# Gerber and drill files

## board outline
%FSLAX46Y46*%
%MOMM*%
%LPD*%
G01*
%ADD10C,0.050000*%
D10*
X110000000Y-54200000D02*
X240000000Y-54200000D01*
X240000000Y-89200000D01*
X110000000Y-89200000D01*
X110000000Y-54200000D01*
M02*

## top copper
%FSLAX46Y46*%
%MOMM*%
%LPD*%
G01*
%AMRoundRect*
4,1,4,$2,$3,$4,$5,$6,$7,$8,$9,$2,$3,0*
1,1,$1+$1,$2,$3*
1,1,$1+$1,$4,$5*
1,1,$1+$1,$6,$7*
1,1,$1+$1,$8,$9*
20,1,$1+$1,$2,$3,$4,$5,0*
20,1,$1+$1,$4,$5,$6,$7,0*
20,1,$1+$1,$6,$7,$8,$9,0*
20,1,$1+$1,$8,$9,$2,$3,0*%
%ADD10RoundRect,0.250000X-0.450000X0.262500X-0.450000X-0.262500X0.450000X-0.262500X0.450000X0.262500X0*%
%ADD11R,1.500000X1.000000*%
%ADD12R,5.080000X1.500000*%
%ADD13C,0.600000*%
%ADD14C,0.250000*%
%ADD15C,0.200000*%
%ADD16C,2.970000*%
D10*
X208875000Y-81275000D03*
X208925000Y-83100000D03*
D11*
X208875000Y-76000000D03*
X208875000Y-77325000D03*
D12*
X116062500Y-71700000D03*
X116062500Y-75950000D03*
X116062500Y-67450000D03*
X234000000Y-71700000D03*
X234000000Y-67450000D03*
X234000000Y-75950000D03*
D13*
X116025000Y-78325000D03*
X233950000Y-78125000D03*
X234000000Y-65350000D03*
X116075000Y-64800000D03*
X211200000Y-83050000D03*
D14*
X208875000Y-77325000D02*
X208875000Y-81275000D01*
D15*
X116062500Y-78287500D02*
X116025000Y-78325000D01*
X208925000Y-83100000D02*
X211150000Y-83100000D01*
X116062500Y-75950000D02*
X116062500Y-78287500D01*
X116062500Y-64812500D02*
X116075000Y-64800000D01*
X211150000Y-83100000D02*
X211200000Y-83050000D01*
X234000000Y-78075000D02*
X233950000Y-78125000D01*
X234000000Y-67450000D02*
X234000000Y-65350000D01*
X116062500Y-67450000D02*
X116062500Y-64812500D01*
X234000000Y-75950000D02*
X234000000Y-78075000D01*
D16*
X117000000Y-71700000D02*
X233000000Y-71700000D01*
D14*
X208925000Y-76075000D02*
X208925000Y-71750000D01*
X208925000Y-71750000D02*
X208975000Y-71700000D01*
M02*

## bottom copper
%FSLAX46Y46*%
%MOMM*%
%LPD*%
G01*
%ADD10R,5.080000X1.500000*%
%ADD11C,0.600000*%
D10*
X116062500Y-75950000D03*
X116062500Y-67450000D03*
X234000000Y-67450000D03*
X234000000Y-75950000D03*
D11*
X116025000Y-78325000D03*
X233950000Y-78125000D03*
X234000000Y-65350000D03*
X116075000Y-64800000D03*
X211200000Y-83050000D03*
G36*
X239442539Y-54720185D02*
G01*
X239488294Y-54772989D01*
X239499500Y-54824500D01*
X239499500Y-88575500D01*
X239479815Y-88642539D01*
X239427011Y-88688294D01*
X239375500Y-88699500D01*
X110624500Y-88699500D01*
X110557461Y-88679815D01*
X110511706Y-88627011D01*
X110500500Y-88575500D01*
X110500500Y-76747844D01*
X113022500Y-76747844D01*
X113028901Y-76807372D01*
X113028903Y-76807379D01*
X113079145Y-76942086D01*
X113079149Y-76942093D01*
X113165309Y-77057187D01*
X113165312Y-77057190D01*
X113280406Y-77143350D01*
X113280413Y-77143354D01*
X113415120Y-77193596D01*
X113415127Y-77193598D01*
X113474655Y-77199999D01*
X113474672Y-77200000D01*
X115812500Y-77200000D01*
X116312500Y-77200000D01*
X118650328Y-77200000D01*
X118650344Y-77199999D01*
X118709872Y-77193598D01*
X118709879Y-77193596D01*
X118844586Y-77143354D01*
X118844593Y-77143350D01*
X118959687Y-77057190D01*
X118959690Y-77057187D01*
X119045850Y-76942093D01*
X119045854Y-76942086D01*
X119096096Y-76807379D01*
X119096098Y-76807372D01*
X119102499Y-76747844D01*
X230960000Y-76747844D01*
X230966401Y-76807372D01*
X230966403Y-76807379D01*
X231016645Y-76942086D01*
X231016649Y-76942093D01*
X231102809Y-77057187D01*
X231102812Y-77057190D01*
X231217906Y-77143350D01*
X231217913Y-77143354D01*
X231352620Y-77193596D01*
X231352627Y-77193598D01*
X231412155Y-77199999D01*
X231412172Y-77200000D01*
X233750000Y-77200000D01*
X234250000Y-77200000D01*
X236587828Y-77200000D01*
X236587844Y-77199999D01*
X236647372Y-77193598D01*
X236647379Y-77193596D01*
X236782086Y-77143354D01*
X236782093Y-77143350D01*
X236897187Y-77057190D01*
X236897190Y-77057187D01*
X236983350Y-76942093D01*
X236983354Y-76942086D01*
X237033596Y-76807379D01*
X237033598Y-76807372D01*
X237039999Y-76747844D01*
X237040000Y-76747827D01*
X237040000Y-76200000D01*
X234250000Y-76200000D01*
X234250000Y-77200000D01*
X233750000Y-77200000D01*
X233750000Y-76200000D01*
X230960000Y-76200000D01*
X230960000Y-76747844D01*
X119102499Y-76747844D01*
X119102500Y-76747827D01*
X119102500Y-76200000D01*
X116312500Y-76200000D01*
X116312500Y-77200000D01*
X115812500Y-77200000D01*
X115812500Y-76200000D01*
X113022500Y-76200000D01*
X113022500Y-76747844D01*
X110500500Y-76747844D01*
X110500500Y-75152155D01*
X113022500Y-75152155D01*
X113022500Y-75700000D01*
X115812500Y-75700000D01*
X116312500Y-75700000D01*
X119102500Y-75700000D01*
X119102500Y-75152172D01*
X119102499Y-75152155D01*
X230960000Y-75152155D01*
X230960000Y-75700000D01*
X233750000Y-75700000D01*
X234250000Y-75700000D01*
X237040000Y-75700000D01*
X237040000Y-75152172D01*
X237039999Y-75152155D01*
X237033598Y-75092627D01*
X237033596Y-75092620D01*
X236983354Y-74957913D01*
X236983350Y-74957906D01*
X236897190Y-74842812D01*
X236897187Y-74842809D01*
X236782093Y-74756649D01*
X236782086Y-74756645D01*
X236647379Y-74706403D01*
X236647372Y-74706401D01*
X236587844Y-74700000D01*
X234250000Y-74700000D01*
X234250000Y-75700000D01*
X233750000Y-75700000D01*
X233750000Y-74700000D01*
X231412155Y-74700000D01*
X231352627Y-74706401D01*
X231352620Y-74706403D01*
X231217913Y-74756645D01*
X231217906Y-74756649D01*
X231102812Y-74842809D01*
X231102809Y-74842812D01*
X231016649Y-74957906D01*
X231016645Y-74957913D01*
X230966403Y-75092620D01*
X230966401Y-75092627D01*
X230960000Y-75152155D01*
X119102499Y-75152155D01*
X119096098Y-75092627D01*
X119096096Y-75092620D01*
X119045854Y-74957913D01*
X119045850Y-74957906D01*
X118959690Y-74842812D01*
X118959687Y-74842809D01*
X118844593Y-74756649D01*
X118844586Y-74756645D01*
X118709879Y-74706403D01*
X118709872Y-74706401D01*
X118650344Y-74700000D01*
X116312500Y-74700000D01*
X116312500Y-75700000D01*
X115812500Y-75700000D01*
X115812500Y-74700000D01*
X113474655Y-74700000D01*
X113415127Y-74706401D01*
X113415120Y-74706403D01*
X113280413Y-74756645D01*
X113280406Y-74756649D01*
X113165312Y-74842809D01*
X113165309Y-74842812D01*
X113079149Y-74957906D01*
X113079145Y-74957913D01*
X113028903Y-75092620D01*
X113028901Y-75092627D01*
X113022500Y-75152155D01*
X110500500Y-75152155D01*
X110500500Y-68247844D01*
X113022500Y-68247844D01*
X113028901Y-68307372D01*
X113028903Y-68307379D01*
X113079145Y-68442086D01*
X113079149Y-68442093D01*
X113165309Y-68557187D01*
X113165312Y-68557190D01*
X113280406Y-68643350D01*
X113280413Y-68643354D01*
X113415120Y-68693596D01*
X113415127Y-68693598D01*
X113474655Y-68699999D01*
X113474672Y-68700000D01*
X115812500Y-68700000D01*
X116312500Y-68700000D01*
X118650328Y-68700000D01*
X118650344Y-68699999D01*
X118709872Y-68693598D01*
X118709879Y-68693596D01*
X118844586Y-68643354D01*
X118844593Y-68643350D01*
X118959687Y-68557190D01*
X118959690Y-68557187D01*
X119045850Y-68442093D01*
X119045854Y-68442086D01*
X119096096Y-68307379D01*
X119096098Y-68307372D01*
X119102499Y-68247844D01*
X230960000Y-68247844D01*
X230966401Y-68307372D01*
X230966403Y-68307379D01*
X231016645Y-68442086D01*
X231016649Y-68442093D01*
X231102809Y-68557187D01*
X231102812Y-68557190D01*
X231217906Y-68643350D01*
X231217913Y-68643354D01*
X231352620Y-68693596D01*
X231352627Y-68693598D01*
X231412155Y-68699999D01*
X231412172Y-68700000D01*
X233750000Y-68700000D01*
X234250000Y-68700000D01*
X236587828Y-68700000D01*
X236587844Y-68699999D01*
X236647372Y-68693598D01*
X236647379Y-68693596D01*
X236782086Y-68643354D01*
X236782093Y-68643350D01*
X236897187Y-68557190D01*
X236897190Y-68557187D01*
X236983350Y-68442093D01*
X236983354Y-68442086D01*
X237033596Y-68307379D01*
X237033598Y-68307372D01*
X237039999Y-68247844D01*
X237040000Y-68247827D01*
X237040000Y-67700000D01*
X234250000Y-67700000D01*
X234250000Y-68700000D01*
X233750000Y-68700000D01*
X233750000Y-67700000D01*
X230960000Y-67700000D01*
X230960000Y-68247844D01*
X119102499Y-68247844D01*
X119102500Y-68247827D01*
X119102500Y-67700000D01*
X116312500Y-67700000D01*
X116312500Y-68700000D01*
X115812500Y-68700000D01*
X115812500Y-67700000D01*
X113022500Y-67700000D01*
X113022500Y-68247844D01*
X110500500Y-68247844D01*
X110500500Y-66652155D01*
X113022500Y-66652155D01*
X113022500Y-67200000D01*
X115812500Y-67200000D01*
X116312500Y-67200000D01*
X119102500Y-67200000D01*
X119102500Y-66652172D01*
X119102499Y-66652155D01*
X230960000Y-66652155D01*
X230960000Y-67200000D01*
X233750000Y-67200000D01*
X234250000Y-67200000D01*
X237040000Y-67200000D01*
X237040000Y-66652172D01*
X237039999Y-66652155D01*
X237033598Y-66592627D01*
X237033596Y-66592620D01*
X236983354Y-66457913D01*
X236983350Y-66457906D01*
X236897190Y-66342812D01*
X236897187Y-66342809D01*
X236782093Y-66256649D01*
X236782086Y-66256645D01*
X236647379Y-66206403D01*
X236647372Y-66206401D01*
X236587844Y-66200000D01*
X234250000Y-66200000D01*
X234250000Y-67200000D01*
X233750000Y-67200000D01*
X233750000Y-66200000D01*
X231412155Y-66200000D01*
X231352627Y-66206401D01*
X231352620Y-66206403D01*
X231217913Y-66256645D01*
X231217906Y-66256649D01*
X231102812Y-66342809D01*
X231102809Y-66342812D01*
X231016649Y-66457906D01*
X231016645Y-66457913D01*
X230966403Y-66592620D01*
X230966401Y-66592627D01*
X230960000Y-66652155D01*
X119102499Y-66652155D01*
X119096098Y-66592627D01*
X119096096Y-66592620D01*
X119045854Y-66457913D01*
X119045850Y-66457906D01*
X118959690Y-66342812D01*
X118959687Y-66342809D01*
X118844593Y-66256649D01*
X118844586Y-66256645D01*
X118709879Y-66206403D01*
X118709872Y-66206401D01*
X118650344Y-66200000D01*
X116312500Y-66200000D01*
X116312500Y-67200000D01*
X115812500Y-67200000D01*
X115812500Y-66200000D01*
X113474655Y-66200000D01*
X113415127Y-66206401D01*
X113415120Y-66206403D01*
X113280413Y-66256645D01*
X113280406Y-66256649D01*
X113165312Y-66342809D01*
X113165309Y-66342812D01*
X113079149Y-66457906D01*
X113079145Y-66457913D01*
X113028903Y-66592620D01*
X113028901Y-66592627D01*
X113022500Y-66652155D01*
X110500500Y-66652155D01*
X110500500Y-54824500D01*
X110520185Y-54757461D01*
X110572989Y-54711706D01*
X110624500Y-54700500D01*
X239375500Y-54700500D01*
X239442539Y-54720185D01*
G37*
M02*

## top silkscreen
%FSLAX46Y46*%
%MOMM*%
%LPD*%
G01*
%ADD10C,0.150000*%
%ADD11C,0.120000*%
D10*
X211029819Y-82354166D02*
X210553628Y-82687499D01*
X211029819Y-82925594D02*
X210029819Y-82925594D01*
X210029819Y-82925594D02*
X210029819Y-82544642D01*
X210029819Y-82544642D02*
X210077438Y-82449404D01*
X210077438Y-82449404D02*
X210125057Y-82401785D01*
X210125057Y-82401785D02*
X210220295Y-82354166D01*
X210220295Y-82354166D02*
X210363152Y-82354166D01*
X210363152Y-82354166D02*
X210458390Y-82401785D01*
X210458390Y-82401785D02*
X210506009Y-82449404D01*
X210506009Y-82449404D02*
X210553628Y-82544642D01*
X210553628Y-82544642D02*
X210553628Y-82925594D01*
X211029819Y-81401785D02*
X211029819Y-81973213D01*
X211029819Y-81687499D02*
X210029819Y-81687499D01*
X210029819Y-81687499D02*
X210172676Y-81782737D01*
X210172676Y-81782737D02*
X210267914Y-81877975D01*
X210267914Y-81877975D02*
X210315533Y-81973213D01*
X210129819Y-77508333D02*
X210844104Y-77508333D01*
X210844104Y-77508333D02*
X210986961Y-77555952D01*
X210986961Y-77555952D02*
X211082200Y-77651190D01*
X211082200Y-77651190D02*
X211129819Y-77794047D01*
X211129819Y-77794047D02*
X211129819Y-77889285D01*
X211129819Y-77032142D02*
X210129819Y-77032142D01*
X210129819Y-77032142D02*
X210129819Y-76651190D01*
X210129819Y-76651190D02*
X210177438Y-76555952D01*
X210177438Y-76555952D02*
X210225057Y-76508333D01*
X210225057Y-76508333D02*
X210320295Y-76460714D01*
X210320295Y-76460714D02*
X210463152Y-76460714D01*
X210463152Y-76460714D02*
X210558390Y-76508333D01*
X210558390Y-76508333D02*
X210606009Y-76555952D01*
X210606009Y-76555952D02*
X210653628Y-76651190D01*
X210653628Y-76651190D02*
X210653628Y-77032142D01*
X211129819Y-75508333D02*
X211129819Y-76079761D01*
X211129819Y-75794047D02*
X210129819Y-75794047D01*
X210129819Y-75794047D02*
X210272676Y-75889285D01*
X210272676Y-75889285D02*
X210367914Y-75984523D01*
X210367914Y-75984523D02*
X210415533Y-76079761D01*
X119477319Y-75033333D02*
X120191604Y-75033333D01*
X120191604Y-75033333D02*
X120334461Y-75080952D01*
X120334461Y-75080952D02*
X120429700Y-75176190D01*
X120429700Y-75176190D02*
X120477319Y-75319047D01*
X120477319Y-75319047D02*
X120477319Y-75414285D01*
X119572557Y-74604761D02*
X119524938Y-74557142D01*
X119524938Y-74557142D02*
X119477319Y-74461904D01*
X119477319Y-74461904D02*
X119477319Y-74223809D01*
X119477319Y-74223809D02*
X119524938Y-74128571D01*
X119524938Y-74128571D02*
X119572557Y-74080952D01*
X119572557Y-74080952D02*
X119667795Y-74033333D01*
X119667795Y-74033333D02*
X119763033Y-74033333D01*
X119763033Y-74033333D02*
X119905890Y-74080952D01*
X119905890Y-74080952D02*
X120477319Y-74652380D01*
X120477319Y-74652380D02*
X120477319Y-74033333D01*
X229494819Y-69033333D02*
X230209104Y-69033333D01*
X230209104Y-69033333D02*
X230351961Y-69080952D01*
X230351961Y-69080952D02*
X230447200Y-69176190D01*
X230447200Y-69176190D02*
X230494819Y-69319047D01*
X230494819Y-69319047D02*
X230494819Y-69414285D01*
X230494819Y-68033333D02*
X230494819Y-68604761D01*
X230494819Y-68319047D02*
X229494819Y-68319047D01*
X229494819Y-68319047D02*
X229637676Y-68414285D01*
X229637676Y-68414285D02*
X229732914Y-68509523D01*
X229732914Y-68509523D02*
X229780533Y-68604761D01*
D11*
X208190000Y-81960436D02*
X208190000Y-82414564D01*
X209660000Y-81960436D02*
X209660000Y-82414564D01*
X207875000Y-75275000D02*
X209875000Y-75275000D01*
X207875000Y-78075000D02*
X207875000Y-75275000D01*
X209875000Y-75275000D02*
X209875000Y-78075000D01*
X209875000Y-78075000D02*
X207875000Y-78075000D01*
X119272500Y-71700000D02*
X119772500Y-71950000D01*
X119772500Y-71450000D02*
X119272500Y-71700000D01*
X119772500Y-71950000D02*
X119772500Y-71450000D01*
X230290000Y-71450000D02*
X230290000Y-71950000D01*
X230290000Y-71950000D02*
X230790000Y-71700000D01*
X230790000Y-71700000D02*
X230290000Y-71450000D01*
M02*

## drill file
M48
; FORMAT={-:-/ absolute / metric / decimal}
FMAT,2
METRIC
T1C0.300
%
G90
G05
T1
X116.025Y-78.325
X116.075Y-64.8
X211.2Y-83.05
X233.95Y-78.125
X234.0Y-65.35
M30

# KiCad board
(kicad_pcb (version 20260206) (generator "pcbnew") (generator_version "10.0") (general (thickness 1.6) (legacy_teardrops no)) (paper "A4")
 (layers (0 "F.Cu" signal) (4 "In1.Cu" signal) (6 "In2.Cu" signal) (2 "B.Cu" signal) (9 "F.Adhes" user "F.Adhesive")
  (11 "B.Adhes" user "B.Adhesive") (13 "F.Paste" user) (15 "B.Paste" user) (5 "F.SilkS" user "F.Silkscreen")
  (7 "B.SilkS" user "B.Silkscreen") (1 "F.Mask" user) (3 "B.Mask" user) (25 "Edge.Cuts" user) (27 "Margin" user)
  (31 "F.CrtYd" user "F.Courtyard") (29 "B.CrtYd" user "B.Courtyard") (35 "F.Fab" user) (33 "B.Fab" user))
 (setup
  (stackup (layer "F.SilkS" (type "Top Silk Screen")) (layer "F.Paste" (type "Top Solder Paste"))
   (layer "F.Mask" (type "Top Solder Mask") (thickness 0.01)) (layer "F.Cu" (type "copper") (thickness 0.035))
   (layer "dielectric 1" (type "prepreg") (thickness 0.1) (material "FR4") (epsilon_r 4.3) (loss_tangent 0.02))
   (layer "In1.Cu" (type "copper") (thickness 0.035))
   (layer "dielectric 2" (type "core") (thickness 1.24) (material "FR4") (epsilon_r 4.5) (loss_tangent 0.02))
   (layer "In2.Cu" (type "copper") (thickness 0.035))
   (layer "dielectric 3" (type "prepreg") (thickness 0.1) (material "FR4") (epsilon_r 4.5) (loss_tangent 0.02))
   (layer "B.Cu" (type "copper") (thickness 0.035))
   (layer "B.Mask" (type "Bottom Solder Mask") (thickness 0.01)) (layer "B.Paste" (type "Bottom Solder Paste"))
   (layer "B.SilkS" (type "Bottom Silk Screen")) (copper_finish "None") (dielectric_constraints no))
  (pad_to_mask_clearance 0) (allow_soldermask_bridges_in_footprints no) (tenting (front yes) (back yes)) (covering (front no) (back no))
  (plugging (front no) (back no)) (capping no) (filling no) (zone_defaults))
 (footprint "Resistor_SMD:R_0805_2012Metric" (layer "F.Cu") (at 208.925 82.1875 -90)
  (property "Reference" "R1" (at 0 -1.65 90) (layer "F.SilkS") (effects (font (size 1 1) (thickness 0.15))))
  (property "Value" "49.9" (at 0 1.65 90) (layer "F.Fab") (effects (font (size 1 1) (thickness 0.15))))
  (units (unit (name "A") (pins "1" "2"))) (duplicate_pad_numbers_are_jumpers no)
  (fp_line (start -0.227064 0.735) (end 0.227064 0.735) (stroke (width 0.12) (type solid)) (layer "F.SilkS"))
  (fp_line (start -0.227064 -0.735) (end 0.227064 -0.735) (stroke (width 0.12) (type solid)) (layer "F.SilkS"))
  (pad "1" smd roundrect (at -0.9125 0.05 270) (size 1.025 1.4) (layers "F.Cu" "F.Mask" "F.Paste") (roundrect_rratio 0.243902)
   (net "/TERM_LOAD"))
  (pad "2" smd roundrect (at 0.9125 0 270) (size 1.025 1.4) (layers "F.Cu" "F.Mask" "F.Paste") (roundrect_rratio 0.243902) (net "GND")))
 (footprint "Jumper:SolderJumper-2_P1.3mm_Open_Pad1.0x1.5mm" (layer "F.Cu") (at 208.875 76.675 -90)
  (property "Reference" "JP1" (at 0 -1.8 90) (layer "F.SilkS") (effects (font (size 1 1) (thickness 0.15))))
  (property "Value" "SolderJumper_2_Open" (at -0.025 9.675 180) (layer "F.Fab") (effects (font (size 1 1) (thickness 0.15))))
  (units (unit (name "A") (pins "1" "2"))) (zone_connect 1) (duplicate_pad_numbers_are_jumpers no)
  (fp_line (start -1.4 1) (end -1.4 -1) (stroke (width 0.12) (type solid)) (layer "F.SilkS"))
  (fp_line (start 1.4 1) (end -1.4 1) (stroke (width 0.12) (type solid)) (layer "F.SilkS"))
  (fp_line (start -1.4 -1) (end 1.4 -1) (stroke (width 0.12) (type solid)) (layer "F.SilkS"))
  (fp_line (start 1.4 -1) (end 1.4 1) (stroke (width 0.12) (type solid)) (layer "F.SilkS"))
  (pad "1" smd rect (at -0.675 0 270) (size 1 1.5) (layers "F.Cu" "F.Mask") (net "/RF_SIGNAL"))
  (pad "2" smd rect (at 0.65 0 270) (size 1 1.5) (layers "F.Cu" "F.Mask") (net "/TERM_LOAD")))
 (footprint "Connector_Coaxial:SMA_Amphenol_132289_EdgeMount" (layer "F.Cu") (at 116.0625 71.7 180)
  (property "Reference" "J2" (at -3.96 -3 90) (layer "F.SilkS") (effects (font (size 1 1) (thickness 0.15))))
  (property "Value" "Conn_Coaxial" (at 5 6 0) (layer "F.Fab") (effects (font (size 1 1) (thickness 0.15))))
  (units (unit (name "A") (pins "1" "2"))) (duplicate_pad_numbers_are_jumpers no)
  (fp_line (start -3.21 0) (end -3.71 -0.25) (stroke (width 0.12) (type solid)) (layer "F.SilkS"))
  (fp_line (start -3.71 0.25) (end -3.21 0) (stroke (width 0.12) (type solid)) (layer "F.SilkS"))
  (fp_line (start -3.71 -0.25) (end -3.71 0.25) (stroke (width 0.12) (type solid)) (layer "F.SilkS"))
  (pad "1" smd rect (at 0 0 270) (size 1.5 5.08) (layers "F.Cu" "F.Mask" "F.Paste") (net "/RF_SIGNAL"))
  (pad "2" smd rect (at 0 -4.25 270) (size 1.5 5.08) (layers "F.Cu" "F.Mask" "F.Paste") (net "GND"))
  (pad "2" smd rect (at 0 -4.25 270) (size 1.5 5.08) (layers "B.Cu" "B.Mask" "B.Paste") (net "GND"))
  (pad "2" smd rect (at 0 4.25 270) (size 1.5 5.08) (layers "F.Cu" "F.Mask" "F.Paste") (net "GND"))
  (pad "2" smd rect (at 0 4.25 270) (size 1.5 5.08) (layers "B.Cu" "B.Mask" "B.Paste") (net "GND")))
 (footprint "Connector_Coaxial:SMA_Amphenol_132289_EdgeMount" (layer "F.Cu") (at 234 71.7)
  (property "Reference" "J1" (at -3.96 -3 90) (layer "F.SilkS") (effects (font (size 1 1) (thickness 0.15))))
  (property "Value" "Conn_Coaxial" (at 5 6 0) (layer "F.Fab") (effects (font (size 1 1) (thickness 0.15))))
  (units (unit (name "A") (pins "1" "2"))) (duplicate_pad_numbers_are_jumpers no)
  (fp_line (start -3.71 -0.25) (end -3.71 0.25) (stroke (width 0.12) (type solid)) (layer "F.SilkS"))
  (fp_line (start -3.71 0.25) (end -3.21 0) (stroke (width 0.12) (type solid)) (layer "F.SilkS"))
  (fp_line (start -3.21 0) (end -3.71 -0.25) (stroke (width 0.12) (type solid)) (layer "F.SilkS"))
  (pad "1" smd rect (at 0 0 90) (size 1.5 5.08) (layers "F.Cu" "F.Mask" "F.Paste") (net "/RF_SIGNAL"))
  (pad "2" smd rect (at 0 -4.25 90) (size 1.5 5.08) (layers "F.Cu" "F.Mask" "F.Paste") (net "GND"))
  (pad "2" smd rect (at 0 -4.25 90) (size 1.5 5.08) (layers "B.Cu" "B.Mask" "B.Paste") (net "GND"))
  (pad "2" smd rect (at 0 4.25 90) (size 1.5 5.08) (layers "F.Cu" "F.Mask" "F.Paste") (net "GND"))
  (pad "2" smd rect (at 0 4.25 90) (size 1.5 5.08) (layers "B.Cu" "B.Mask" "B.Paste") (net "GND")))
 (gr_rect (start 110 54.2) (end 240 89.2) (stroke (width 0.05) (type solid)) (fill no) (layer "Edge.Cuts"))
 (segment (start 208.875 77.325) (end 208.875 81.275) (width 0.25) (layer "F.Cu") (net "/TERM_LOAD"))
 (segment (start 116.0625 78.2875) (end 116.025 78.325) (width 0.2) (layer "F.Cu") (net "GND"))
 (segment (start 208.925 83.1) (end 211.15 83.1) (width 0.2) (layer "F.Cu") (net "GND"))
 (segment (start 116.0625 75.95) (end 116.0625 78.2875) (width 0.2) (layer "F.Cu") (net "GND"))
 (segment (start 116.0625 64.8125) (end 116.075 64.8) (width 0.2) (layer "F.Cu") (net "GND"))
 (segment (start 211.15 83.1) (end 211.2 83.05) (width 0.2) (layer "F.Cu") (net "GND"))
 (segment (start 234 78.075) (end 233.95 78.125) (width 0.2) (layer "F.Cu") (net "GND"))
 (segment (start 234 67.45) (end 234 65.35) (width 0.2) (layer "F.Cu") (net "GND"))
 (segment (start 116.0625 67.45) (end 116.0625 64.8125) (width 0.2) (layer "F.Cu") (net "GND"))
 (segment (start 234 75.95) (end 234 78.075) (width 0.2) (layer "F.Cu") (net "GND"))
 (via (at 116.025 78.325) (size 0.6) (drill 0.3) (layers "F.Cu" "B.Cu") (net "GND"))
 (via (at 233.95 78.125) (size 0.6) (drill 0.3) (layers "F.Cu" "B.Cu") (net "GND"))
 (via (at 234 65.35) (size 0.6) (drill 0.3) (layers "F.Cu" "B.Cu") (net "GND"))
 (via (at 116.075 64.8) (size 0.6) (drill 0.3) (layers "F.Cu" "B.Cu") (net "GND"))
 (via (at 211.2 83.05) (size 0.6) (drill 0.3) (layers "F.Cu" "B.Cu") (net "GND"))
 (segment (start 117 71.7) (end 233 71.7) (width 2.97) (layer "F.Cu") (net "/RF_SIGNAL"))
 (segment (start 208.925 76.075) (end 208.925 71.75) (width 0.25) (layer "F.Cu") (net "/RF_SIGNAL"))
 (segment (start 208.925 71.75) (end 208.975 71.7) (width 0.25) (layer "F.Cu") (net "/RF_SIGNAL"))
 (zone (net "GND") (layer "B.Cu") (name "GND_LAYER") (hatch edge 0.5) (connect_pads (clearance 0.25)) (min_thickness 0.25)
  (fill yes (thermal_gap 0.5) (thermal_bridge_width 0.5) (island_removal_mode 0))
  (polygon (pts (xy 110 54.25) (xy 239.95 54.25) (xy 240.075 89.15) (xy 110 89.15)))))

